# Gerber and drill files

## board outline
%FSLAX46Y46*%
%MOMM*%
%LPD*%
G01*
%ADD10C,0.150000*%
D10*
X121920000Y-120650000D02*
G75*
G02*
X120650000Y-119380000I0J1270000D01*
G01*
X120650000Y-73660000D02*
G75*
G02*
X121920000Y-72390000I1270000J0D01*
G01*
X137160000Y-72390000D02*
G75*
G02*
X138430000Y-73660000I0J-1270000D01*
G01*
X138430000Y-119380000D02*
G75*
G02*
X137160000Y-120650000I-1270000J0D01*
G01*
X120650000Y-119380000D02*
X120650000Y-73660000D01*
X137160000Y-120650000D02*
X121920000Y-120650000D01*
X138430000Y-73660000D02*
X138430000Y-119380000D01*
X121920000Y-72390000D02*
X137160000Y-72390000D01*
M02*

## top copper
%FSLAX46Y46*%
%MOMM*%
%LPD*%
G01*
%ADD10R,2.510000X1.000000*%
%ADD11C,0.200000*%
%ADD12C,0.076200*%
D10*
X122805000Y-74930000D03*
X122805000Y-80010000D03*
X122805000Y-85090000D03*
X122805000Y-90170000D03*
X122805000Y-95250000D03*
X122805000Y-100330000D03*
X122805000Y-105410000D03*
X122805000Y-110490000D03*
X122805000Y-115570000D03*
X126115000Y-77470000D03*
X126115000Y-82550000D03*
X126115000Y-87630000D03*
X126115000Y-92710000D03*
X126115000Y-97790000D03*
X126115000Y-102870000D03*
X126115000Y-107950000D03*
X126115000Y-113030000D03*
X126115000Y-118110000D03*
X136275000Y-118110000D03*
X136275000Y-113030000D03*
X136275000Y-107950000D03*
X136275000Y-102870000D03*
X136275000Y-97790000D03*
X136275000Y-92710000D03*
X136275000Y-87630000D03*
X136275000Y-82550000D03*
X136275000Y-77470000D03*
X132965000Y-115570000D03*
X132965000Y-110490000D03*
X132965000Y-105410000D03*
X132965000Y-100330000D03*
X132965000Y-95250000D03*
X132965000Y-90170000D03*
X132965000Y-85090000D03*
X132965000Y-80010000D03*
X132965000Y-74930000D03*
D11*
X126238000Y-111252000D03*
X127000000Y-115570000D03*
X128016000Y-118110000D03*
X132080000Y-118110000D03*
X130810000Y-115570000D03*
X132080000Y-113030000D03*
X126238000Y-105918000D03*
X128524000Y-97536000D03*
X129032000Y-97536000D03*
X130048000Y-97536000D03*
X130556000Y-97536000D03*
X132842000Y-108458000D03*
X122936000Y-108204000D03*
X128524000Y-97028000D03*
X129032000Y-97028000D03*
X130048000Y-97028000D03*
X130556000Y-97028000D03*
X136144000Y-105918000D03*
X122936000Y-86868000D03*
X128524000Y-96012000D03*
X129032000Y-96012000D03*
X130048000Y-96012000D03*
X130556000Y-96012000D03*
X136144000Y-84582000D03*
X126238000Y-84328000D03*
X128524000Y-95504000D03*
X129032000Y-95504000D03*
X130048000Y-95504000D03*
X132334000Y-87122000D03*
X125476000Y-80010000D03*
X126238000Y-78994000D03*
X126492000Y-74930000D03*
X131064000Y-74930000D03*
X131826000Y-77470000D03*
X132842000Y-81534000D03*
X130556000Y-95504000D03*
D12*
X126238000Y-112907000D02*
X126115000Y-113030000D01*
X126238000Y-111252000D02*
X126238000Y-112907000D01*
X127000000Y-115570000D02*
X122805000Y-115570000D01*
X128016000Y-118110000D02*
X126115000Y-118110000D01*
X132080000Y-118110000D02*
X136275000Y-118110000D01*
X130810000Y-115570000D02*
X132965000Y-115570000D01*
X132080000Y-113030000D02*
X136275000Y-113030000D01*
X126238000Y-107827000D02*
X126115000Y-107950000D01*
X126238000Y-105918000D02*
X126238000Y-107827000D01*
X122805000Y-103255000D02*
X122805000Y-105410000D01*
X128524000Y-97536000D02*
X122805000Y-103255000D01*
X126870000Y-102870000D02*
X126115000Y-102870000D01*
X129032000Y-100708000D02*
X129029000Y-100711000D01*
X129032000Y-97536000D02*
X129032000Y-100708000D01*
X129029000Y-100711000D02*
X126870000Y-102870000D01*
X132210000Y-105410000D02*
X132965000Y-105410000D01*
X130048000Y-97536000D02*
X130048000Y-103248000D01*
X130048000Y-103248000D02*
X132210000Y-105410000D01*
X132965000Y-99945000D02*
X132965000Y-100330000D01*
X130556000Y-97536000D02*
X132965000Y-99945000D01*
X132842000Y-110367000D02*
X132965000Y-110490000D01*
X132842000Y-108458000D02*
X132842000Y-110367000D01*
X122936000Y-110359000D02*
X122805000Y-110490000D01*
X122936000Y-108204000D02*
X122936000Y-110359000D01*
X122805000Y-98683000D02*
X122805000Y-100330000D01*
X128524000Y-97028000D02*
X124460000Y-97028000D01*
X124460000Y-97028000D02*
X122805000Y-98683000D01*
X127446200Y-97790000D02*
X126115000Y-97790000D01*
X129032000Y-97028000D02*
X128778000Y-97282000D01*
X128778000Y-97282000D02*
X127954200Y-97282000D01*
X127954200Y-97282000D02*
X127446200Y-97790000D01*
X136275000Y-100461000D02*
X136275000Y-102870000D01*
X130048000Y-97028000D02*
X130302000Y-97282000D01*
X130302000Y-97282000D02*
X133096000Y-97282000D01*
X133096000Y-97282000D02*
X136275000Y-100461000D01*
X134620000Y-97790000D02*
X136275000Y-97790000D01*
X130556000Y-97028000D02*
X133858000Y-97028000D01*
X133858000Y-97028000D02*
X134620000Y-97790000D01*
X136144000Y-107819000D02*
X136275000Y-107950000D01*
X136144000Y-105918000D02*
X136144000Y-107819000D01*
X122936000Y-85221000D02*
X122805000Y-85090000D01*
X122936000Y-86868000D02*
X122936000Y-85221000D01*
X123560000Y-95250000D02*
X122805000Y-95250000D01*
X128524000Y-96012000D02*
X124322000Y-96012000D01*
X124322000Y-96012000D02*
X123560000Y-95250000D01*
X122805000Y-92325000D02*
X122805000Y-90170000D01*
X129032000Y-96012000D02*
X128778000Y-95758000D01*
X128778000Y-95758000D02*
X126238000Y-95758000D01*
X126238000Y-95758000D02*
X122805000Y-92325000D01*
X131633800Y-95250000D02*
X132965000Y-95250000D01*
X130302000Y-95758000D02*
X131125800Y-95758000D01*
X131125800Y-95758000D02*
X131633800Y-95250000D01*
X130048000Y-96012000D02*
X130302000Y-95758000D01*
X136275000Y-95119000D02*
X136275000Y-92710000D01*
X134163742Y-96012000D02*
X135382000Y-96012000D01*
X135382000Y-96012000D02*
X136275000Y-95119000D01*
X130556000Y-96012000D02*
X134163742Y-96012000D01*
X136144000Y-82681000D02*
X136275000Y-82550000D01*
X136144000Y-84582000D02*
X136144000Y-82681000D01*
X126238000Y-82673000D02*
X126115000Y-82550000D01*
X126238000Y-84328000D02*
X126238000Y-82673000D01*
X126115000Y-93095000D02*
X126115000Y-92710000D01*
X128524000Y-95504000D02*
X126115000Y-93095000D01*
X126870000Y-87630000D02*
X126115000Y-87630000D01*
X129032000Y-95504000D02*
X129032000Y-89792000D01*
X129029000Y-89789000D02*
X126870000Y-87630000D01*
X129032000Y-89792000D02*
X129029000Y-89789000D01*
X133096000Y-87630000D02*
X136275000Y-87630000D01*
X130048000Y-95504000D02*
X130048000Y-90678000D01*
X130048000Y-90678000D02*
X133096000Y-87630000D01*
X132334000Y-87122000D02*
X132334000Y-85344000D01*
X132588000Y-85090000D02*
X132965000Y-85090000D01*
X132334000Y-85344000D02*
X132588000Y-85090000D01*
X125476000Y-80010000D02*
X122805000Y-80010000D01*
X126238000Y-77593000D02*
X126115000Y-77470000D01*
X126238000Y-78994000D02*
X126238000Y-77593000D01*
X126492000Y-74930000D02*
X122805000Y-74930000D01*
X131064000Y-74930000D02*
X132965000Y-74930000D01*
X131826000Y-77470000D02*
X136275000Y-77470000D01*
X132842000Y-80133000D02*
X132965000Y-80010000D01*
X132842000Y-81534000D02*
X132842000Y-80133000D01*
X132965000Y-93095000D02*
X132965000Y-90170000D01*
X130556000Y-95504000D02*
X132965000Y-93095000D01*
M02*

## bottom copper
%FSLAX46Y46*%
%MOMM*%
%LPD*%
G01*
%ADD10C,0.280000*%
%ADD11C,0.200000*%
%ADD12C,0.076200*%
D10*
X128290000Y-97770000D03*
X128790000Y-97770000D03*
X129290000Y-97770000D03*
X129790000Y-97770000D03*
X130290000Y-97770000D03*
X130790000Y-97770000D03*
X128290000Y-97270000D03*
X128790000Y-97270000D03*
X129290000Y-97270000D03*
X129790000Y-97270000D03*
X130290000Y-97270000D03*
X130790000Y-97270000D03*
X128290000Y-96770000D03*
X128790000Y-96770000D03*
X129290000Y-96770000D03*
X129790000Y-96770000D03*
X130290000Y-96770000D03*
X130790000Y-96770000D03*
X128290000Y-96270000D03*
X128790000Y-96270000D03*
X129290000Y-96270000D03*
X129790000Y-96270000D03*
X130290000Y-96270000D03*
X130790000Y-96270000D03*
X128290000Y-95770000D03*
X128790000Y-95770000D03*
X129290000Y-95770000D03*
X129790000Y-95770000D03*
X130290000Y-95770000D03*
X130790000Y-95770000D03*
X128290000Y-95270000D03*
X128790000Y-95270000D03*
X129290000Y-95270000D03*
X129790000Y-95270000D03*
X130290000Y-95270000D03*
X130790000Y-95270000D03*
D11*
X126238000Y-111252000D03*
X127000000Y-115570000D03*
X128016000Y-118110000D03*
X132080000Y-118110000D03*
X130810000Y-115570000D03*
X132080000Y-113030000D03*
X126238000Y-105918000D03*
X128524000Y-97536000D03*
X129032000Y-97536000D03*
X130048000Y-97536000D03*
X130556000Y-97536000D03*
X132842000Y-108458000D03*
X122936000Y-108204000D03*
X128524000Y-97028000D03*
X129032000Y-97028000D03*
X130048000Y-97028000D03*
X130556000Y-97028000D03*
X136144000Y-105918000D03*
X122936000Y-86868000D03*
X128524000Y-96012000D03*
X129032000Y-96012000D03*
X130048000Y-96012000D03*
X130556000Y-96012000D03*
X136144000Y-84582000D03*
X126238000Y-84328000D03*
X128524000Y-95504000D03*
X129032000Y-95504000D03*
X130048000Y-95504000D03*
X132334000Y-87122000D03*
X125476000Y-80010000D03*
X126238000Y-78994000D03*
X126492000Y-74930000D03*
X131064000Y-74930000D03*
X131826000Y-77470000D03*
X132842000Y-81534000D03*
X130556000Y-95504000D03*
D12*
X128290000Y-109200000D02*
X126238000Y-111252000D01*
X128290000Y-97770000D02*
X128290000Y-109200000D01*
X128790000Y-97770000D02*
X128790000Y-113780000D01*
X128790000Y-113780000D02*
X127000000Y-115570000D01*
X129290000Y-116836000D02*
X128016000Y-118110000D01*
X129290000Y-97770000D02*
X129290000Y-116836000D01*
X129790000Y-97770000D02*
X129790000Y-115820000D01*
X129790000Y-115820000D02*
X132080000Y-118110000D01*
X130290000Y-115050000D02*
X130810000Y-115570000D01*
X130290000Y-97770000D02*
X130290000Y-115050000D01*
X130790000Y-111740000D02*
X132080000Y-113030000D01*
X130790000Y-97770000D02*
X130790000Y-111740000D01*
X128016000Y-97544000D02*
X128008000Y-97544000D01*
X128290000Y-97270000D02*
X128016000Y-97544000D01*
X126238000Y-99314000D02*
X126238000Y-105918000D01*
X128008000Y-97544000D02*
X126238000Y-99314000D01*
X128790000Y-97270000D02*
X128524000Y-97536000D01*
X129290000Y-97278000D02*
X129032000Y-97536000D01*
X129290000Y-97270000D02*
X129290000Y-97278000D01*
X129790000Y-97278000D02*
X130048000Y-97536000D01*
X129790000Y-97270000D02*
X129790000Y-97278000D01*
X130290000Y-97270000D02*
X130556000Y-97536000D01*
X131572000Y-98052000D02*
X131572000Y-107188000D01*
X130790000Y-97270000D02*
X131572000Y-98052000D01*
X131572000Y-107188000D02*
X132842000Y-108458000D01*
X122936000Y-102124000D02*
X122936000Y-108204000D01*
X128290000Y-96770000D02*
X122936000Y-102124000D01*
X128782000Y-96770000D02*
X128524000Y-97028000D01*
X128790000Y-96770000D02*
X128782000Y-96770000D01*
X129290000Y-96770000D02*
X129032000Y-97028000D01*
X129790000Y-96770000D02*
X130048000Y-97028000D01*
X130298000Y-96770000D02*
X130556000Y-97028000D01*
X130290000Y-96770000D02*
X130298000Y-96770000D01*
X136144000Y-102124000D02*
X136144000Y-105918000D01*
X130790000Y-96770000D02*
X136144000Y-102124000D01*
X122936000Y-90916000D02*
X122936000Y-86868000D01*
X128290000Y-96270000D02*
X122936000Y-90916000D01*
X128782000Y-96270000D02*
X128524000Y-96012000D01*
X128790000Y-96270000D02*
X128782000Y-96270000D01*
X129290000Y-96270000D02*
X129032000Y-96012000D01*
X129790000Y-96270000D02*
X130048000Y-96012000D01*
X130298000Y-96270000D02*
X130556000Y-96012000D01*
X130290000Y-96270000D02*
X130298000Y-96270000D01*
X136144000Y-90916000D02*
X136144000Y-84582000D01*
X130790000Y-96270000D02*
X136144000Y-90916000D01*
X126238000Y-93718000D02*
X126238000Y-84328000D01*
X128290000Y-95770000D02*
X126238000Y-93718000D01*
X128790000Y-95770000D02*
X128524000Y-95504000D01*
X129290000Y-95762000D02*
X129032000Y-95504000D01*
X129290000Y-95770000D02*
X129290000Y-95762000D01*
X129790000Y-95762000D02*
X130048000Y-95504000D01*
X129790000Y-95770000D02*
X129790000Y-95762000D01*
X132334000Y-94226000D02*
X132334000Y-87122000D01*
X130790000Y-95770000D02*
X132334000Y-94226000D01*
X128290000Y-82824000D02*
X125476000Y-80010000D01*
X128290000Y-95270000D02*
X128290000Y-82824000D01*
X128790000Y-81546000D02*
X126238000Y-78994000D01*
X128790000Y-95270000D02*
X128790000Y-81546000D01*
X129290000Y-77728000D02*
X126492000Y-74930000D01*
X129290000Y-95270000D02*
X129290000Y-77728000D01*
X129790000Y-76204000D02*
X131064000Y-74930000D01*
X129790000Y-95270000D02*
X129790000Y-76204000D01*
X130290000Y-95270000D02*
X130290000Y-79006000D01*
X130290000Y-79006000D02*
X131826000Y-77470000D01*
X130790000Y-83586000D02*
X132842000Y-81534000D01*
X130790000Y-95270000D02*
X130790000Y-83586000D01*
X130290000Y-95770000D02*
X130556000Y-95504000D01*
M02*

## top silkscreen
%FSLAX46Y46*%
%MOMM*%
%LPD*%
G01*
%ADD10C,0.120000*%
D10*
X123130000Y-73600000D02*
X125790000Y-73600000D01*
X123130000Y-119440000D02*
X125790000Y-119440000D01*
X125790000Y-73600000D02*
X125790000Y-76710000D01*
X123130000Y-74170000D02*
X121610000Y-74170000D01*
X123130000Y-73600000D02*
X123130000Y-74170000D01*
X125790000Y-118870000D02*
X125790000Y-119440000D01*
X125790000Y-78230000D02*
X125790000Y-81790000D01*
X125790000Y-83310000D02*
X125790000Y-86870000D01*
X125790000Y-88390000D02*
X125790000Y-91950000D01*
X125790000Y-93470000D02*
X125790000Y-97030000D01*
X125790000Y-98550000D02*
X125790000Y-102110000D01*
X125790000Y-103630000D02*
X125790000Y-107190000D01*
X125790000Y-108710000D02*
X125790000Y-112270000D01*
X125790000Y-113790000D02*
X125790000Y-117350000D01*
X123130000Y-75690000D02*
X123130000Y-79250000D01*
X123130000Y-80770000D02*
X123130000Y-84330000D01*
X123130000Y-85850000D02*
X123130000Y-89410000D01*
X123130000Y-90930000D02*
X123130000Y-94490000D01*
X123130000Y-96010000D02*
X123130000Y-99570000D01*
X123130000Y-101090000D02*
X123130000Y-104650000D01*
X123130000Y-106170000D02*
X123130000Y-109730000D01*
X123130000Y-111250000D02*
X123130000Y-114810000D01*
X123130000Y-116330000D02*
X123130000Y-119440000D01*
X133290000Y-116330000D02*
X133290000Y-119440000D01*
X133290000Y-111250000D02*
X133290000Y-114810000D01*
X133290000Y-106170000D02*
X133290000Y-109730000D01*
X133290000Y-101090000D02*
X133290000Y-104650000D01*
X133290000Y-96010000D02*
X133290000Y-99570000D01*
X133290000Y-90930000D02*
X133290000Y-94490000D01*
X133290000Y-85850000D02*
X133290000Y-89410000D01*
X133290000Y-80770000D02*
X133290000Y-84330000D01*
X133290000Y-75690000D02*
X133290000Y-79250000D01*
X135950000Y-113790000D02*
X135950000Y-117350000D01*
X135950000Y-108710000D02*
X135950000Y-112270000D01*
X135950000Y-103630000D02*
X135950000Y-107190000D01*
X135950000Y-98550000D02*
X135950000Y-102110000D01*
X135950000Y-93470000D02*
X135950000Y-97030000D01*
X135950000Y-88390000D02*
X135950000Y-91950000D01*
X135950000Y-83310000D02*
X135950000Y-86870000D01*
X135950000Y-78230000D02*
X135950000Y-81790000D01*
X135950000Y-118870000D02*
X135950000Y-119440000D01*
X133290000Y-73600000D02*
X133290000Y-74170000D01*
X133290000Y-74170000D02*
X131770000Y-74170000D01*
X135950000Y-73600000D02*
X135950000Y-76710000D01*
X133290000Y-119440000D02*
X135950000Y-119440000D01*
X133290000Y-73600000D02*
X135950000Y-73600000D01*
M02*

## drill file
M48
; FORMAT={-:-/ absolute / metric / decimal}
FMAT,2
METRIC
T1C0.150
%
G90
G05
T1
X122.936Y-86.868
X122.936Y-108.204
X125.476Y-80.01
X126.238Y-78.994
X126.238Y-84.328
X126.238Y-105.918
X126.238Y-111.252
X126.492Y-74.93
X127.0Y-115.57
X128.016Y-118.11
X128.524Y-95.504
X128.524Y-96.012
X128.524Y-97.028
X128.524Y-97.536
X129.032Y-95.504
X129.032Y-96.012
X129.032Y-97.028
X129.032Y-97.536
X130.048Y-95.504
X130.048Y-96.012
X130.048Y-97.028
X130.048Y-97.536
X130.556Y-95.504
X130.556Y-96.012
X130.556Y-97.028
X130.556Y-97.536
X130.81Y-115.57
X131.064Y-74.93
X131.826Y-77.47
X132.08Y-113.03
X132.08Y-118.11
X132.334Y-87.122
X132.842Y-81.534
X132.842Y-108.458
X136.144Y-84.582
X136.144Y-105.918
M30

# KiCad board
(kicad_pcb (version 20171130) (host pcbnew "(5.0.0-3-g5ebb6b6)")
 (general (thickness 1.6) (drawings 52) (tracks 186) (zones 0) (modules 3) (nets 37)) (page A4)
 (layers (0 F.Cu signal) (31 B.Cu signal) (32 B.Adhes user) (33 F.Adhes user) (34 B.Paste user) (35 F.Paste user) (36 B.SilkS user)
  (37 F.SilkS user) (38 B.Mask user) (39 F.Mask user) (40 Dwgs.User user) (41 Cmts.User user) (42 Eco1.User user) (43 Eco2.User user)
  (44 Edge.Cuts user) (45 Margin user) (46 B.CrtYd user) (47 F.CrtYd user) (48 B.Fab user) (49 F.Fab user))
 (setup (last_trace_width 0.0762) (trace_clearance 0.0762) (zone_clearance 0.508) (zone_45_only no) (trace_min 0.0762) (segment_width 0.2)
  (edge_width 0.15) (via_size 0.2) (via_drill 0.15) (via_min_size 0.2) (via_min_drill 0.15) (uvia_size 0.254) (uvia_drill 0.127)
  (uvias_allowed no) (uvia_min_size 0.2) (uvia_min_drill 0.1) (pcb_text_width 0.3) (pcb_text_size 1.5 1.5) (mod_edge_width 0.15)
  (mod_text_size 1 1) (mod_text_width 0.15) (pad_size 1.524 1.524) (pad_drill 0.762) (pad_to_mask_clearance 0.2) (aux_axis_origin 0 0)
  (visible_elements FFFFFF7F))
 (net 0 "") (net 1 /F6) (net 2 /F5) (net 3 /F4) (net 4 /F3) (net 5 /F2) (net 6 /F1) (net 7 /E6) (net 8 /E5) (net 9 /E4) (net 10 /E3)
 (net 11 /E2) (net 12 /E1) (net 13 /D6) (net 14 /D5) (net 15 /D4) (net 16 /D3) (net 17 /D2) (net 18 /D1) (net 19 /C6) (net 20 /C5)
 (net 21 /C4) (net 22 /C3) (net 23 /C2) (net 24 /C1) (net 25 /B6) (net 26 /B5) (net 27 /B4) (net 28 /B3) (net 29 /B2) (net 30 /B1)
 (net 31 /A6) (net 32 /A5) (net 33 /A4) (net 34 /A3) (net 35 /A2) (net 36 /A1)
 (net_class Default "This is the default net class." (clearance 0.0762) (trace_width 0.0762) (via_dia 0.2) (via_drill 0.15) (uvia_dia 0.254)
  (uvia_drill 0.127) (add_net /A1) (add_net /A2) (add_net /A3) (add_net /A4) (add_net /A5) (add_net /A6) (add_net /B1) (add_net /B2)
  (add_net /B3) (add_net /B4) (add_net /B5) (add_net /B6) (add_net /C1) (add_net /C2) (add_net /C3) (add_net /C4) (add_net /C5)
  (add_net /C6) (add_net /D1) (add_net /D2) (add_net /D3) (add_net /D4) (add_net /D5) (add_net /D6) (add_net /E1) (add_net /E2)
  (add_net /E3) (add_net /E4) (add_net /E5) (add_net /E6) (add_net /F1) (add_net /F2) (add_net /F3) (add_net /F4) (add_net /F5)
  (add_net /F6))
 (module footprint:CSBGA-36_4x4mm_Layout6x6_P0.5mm (layer B.Cu) (at 129.54 96.52 180)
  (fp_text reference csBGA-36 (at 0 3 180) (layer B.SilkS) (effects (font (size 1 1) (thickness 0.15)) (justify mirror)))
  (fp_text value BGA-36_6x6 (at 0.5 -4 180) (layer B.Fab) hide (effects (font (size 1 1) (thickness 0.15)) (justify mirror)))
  (pad F6 smd circle (at 1.25 -1.25 180) (size 0.28 0.28) (layers B.Cu B.Paste B.Mask) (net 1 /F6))
  (pad F5 smd circle (at 0.75 -1.25 180) (size 0.28 0.28) (layers B.Cu B.Paste B.Mask) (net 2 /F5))
  (pad F4 smd circle (at 0.25 -1.25 180) (size 0.28 0.28) (layers B.Cu B.Paste B.Mask) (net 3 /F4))
  (pad F3 smd circle (at -0.25 -1.25 180) (size 0.28 0.28) (layers B.Cu B.Paste B.Mask) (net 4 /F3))
  (pad F2 smd circle (at -0.75 -1.25 180) (size 0.28 0.28) (layers B.Cu B.Paste B.Mask) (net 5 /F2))
  (pad F1 smd circle (at -1.25 -1.25 180) (size 0.28 0.28) (layers B.Cu B.Paste B.Mask) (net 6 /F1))
  (pad E6 smd circle (at 1.25 -0.75 180) (size 0.28 0.28) (layers B.Cu B.Paste B.Mask) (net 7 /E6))
  (pad E5 smd circle (at 0.75 -0.75 180) (size 0.28 0.28) (layers B.Cu B.Paste B.Mask) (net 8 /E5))
  (pad E4 smd circle (at 0.25 -0.75 180) (size 0.28 0.28) (layers B.Cu B.Paste B.Mask) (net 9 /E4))
  (pad E3 smd circle (at -0.25 -0.75 180) (size 0.28 0.28) (layers B.Cu B.Paste B.Mask) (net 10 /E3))
  (pad E2 smd circle (at -0.75 -0.75 180) (size 0.28 0.28) (layers B.Cu B.Paste B.Mask) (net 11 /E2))
  (pad E1 smd circle (at -1.25 -0.75 180) (size 0.28 0.28) (layers B.Cu B.Paste B.Mask) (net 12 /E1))
  (pad D6 smd circle (at 1.25 -0.25 180) (size 0.28 0.28) (layers B.Cu B.Paste B.Mask) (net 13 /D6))
  (pad D5 smd circle (at 0.75 -0.25 180) (size 0.28 0.28) (layers B.Cu B.Paste B.Mask) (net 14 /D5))
  (pad D4 smd circle (at 0.25 -0.25 180) (size 0.28 0.28) (layers B.Cu B.Paste B.Mask) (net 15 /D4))
  (pad D3 smd circle (at -0.25 -0.25 180) (size 0.28 0.28) (layers B.Cu B.Paste B.Mask) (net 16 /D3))
  (pad D2 smd circle (at -0.75 -0.25 180) (size 0.28 0.28) (layers B.Cu B.Paste B.Mask) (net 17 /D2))
  (pad D1 smd circle (at -1.25 -0.25 180) (size 0.28 0.28) (layers B.Cu B.Paste B.Mask) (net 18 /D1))
  (pad C6 smd circle (at 1.25 0.25 180) (size 0.28 0.28) (layers B.Cu B.Paste B.Mask) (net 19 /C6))
  (pad C5 smd circle (at 0.75 0.25 180) (size 0.28 0.28) (layers B.Cu B.Paste B.Mask) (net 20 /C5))
  (pad C4 smd circle (at 0.25 0.25 180) (size 0.28 0.28) (layers B.Cu B.Paste B.Mask) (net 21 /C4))
  (pad C3 smd circle (at -0.25 0.25 180) (size 0.28 0.28) (layers B.Cu B.Paste B.Mask) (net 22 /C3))
  (pad C2 smd circle (at -0.75 0.25 180) (size 0.28 0.28) (layers B.Cu B.Paste B.Mask) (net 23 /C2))
  (pad C1 smd circle (at -1.25 0.25 180) (size 0.28 0.28) (layers B.Cu B.Paste B.Mask) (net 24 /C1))
  (pad B6 smd circle (at 1.25 0.75 180) (size 0.28 0.28) (layers B.Cu B.Paste B.Mask) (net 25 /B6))
  (pad B5 smd circle (at 0.75 0.75 180) (size 0.28 0.28) (layers B.Cu B.Paste B.Mask) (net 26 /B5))
  (pad B4 smd circle (at 0.25 0.75 180) (size 0.28 0.28) (layers B.Cu B.Paste B.Mask) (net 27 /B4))
  (pad B3 smd circle (at -0.25 0.75 180) (size 0.28 0.28) (layers B.Cu B.Paste B.Mask) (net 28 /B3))
  (pad B2 smd circle (at -0.75 0.75 180) (size 0.28 0.28) (layers B.Cu B.Paste B.Mask) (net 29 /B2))
  (pad B1 smd circle (at -1.25 0.75 180) (size 0.28 0.28) (layers B.Cu B.Paste B.Mask) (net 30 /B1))
  (pad A6 smd circle (at 1.25 1.25 180) (size 0.28 0.28) (layers B.Cu B.Paste B.Mask) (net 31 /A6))
  (pad A5 smd circle (at 0.75 1.25 180) (size 0.28 0.28) (layers B.Cu B.Paste B.Mask) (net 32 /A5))
  (pad A4 smd circle (at 0.25 1.25 180) (size 0.28 0.28) (layers B.Cu B.Paste B.Mask) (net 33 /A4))
  (pad A3 smd circle (at -0.25 1.25 180) (size 0.28 0.28) (layers B.Cu B.Paste B.Mask) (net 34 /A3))
  (pad A2 smd circle (at -0.75 1.25 180) (size 0.28 0.28) (layers B.Cu B.Paste B.Mask) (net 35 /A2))
  (pad A1 smd circle (at -1.25 1.25 180) (size 0.28 0.28) (layers B.Cu B.Paste B.Mask) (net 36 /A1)))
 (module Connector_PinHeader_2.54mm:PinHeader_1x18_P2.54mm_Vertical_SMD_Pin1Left (layer F.Cu) (at 124.46 96.52)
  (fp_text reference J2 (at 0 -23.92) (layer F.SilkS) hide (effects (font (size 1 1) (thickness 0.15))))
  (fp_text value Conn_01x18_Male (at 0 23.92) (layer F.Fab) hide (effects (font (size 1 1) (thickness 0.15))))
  (fp_line (start -1.33 -22.92) (end 1.33 -22.92) (layer F.SilkS) (width 0.12))
  (fp_line (start -1.33 22.92) (end 1.33 22.92) (layer F.SilkS) (width 0.12))
  (fp_line (start 1.33 -22.92) (end 1.33 -19.81) (layer F.SilkS) (width 0.12))
  (fp_line (start -1.33 -22.35) (end -2.85 -22.35) (layer F.SilkS) (width 0.12))
  (fp_line (start -1.33 -22.92) (end -1.33 -22.35) (layer F.SilkS) (width 0.12))
  (fp_line (start 1.33 22.35) (end 1.33 22.92) (layer F.SilkS) (width 0.12))
  (fp_line (start 1.33 -18.29) (end 1.33 -14.73) (layer F.SilkS) (width 0.12))
  (fp_line (start 1.33 -13.21) (end 1.33 -9.65) (layer F.SilkS) (width 0.12))
  (fp_line (start 1.33 -8.13) (end 1.33 -4.57) (layer F.SilkS) (width 0.12))
  (fp_line (start 1.33 -3.05) (end 1.33 0.51) (layer F.SilkS) (width 0.12))
  (fp_line (start 1.33 2.03) (end 1.33 5.59) (layer F.SilkS) (width 0.12))
  (fp_line (start 1.33 7.11) (end 1.33 10.67) (layer F.SilkS) (width 0.12))
  (fp_line (start 1.33 12.19) (end 1.33 15.75) (layer F.SilkS) (width 0.12))
  (fp_line (start 1.33 17.27) (end 1.33 20.83) (layer F.SilkS) (width 0.12))
  (fp_line (start -1.33 -20.83) (end -1.33 -17.27) (layer F.SilkS) (width 0.12))
  (fp_line (start -1.33 -15.75) (end -1.33 -12.19) (layer F.SilkS) (width 0.12))
  (fp_line (start -1.33 -10.67) (end -1.33 -7.11) (layer F.SilkS) (width 0.12))
  (fp_line (start -1.33 -5.59) (end -1.33 -2.03) (layer F.SilkS) (width 0.12))
  (fp_line (start -1.33 -0.51) (end -1.33 3.05) (layer F.SilkS) (width 0.12))
  (fp_line (start -1.33 4.57) (end -1.33 8.13) (layer F.SilkS) (width 0.12))
  (fp_line (start -1.33 9.65) (end -1.33 13.21) (layer F.SilkS) (width 0.12))
  (fp_line (start -1.33 14.73) (end -1.33 18.29) (layer F.SilkS) (width 0.12))
  (fp_line (start -1.33 19.81) (end -1.33 22.92) (layer F.SilkS) (width 0.12))
  (pad 1 smd rect (at -1.655 -21.59) (size 2.51 1) (layers F.Cu F.Paste F.Mask) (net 33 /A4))
  (pad 3 smd rect (at -1.655 -16.51) (size 2.51 1) (layers F.Cu F.Paste F.Mask) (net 31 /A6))
  (pad 5 smd rect (at -1.655 -11.43) (size 2.51 1) (layers F.Cu F.Paste F.Mask) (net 19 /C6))
  (pad 7 smd rect (at -1.655 -6.35) (size 2.51 1) (layers F.Cu F.Paste F.Mask) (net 21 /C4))
  (pad 9 smd rect (at -1.655 -1.27) (size 2.51 1) (layers F.Cu F.Paste F.Mask) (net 20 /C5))
  (pad 11 smd rect (at -1.655 3.81) (size 2.51 1) (layers F.Cu F.Paste F.Mask) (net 14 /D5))
  (pad 13 smd rect (at -1.655 8.89) (size 2.51 1) (layers F.Cu F.Paste F.Mask) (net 8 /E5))
  (pad 15 smd rect (at -1.655 13.97) (size 2.51 1) (layers F.Cu F.Paste F.Mask) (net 13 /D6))
  (pad 17 smd rect (at -1.655 19.05) (size 2.51 1) (layers F.Cu F.Paste F.Mask) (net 2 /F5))
  (pad 2 smd rect (at 1.655 -19.05) (size 2.51 1) (layers F.Cu F.Paste F.Mask) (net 32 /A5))
  (pad 4 smd rect (at 1.655 -13.97) (size 2.51 1) (layers F.Cu F.Paste F.Mask) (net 25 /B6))
  (pad 6 smd rect (at 1.655 -8.89) (size 2.51 1) (layers F.Cu F.Paste F.Mask) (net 27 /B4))
  (pad 8 smd rect (at 1.655 -3.81) (size 2.51 1) (layers F.Cu F.Paste F.Mask) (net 26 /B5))
  (pad 10 smd rect (at 1.655 1.27) (size 2.51 1) (layers F.Cu F.Paste F.Mask) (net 15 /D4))
  (pad 12 smd rect (at 1.655 6.35) (size 2.51 1) (layers F.Cu F.Paste F.Mask) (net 9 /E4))
  (pad 14 smd rect (at 1.655 11.43) (size 2.51 1) (layers F.Cu F.Paste F.Mask) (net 7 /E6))
  (pad 16 smd rect (at 1.655 16.51) (size 2.51 1) (layers F.Cu F.Paste F.Mask) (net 1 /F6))
  (pad 18 smd rect (at 1.655 21.59) (size 2.51 1) (layers F.Cu F.Paste F.Mask) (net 3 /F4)))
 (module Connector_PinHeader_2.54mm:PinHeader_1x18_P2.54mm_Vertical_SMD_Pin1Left (layer F.Cu) (at 134.62 96.52)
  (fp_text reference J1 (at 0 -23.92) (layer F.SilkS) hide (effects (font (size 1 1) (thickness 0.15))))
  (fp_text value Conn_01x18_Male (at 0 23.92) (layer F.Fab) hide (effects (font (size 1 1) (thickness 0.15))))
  (fp_line (start -1.33 19.81) (end -1.33 22.92) (layer F.SilkS) (width 0.12))
  (fp_line (start -1.33 14.73) (end -1.33 18.29) (layer F.SilkS) (width 0.12))
  (fp_line (start -1.33 9.65) (end -1.33 13.21) (layer F.SilkS) (width 0.12))
  (fp_line (start -1.33 4.57) (end -1.33 8.13) (layer F.SilkS) (width 0.12))
  (fp_line (start -1.33 -0.51) (end -1.33 3.05) (layer F.SilkS) (width 0.12))
  (fp_line (start -1.33 -5.59) (end -1.33 -2.03) (layer F.SilkS) (width 0.12))
  (fp_line (start -1.33 -10.67) (end -1.33 -7.11) (layer F.SilkS) (width 0.12))
  (fp_line (start -1.33 -15.75) (end -1.33 -12.19) (layer F.SilkS) (width 0.12))
  (fp_line (start -1.33 -20.83) (end -1.33 -17.27) (layer F.SilkS) (width 0.12))
  (fp_line (start 1.33 17.27) (end 1.33 20.83) (layer F.SilkS) (width 0.12))
  (fp_line (start 1.33 12.19) (end 1.33 15.75) (layer F.SilkS) (width 0.12))
  (fp_line (start 1.33 7.11) (end 1.33 10.67) (layer F.SilkS) (width 0.12))
  (fp_line (start 1.33 2.03) (end 1.33 5.59) (layer F.SilkS) (width 0.12))
  (fp_line (start 1.33 -3.05) (end 1.33 0.51) (layer F.SilkS) (width 0.12))
  (fp_line (start 1.33 -8.13) (end 1.33 -4.57) (layer F.SilkS) (width 0.12))
  (fp_line (start 1.33 -13.21) (end 1.33 -9.65) (layer F.SilkS) (width 0.12))
  (fp_line (start 1.33 -18.29) (end 1.33 -14.73) (layer F.SilkS) (width 0.12))
  (fp_line (start 1.33 22.35) (end 1.33 22.92) (layer F.SilkS) (width 0.12))
  (fp_line (start -1.33 -22.92) (end -1.33 -22.35) (layer F.SilkS) (width 0.12))
  (fp_line (start -1.33 -22.35) (end -2.85 -22.35) (layer F.SilkS) (width 0.12))
  (fp_line (start 1.33 -22.92) (end 1.33 -19.81) (layer F.SilkS) (width 0.12))
  (fp_line (start -1.33 22.92) (end 1.33 22.92) (layer F.SilkS) (width 0.12))
  (fp_line (start -1.33 -22.92) (end 1.33 -22.92) (layer F.SilkS) (width 0.12))
  (pad 18 smd rect (at 1.655 21.59) (size 2.51 1) (layers F.Cu F.Paste F.Mask) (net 4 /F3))
  (pad 16 smd rect (at 1.655 16.51) (size 2.51 1) (layers F.Cu F.Paste F.Mask) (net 6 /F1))
  (pad 14 smd rect (at 1.655 11.43) (size 2.51 1) (layers F.Cu F.Paste F.Mask) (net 18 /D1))
  (pad 12 smd rect (at 1.655 6.35) (size 2.51 1) (layers F.Cu F.Paste F.Mask) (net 16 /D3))
  (pad 10 smd rect (at 1.655 1.27) (size 2.51 1) (layers F.Cu F.Paste F.Mask) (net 17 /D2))
  (pad 8 smd rect (at 1.655 -3.81) (size 2.51 1) (layers F.Cu F.Paste F.Mask) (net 23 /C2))
  (pad 6 smd rect (at 1.655 -8.89) (size 2.51 1) (layers F.Cu F.Paste F.Mask) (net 28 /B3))
  (pad 4 smd rect (at 1.655 -13.97) (size 2.51 1) (layers F.Cu F.Paste F.Mask) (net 24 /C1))
  (pad 2 smd rect (at 1.655 -19.05) (size 2.51 1) (layers F.Cu F.Paste F.Mask) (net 35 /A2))
  (pad 17 smd rect (at -1.655 19.05) (size 2.51 1) (layers F.Cu F.Paste F.Mask) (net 5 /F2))
  (pad 15 smd rect (at -1.655 13.97) (size 2.51 1) (layers F.Cu F.Paste F.Mask) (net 12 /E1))
  (pad 13 smd rect (at -1.655 8.89) (size 2.51 1) (layers F.Cu F.Paste F.Mask) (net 10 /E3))
  (pad 11 smd rect (at -1.655 3.81) (size 2.51 1) (layers F.Cu F.Paste F.Mask) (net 11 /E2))
  (pad 9 smd rect (at -1.655 -1.27) (size 2.51 1) (layers F.Cu F.Paste F.Mask) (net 22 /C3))
  (pad 7 smd rect (at -1.655 -6.35) (size 2.51 1) (layers F.Cu F.Paste F.Mask) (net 29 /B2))
  (pad 5 smd rect (at -1.655 -11.43) (size 2.51 1) (layers F.Cu F.Paste F.Mask) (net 30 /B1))
  (pad 3 smd rect (at -1.655 -16.51) (size 2.51 1) (layers F.Cu F.Paste F.Mask) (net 36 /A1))
  (pad 1 smd rect (at -1.655 -21.59) (size 2.51 1) (layers F.Cu F.Paste F.Mask) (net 34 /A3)))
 (gr_arc (start 121.92 119.38) (end 120.65 119.38) (angle -90) (layer Edge.Cuts) (width 0.15))
 (gr_arc (start 121.92 73.66) (end 121.92 72.39) (angle -90) (layer Edge.Cuts) (width 0.15))
 (gr_arc (start 137.16 73.66) (end 138.43 73.66) (angle -90) (layer Edge.Cuts) (width 0.15))
 (gr_arc (start 137.16 119.38) (end 137.16 120.65) (angle -90) (layer Edge.Cuts) (width 0.15))
 (gr_line (start 120.65 119.38) (end 120.65 73.66) (layer Edge.Cuts) (width 0.15))
 (gr_line (start 137.16 120.65) (end 121.92 120.65) (layer Edge.Cuts) (width 0.15))
 (gr_line (start 138.43 73.66) (end 138.43 119.38) (layer Edge.Cuts) (width 0.15))
 (gr_line (start 121.92 72.39) (end 137.16 72.39) (layer Edge.Cuts) (width 0.15))
 (via (at 126.238 111.252) (size 0.2) (drill 0.15) (layers F.Cu B.Cu) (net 1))
 (segment (start 128.29 109.2) (end 126.238 111.252) (width 0.0762) (layer B.Cu) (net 1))
 (segment (start 128.29 97.77) (end 128.29 109.2) (width 0.0762) (layer B.Cu) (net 1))
 (segment (start 126.238 112.907) (end 126.115 113.03) (width 0.0762) (layer F.Cu) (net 1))
 (segment (start 126.238 111.252) (end 126.238 112.907) (width 0.0762) (layer F.Cu) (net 1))
 (segment (start 128.79 97.77) (end 128.79 113.78) (width 0.0762) (layer B.Cu) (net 2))
 (via (at 127 115.57) (size 0.2) (drill 0.15) (layers F.Cu B.Cu) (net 2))
 (segment (start 128.79 113.78) (end 127 115.57) (width 0.0762) (layer B.Cu) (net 2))
 (segment (start 127 115.57) (end 122.805 115.57) (width 0.0762) (layer F.Cu) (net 2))
 (segment (start 129.29 116.836) (end 128.016 118.11) (width 0.0762) (layer B.Cu) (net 3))
 (via (at 128.016 118.11) (size 0.2) (drill 0.15) (layers F.Cu B.Cu) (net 3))
 (segment (start 129.29 97.77) (end 129.29 116.836) (width 0.0762) (layer B.Cu) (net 3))
 (segment (start 128.016 118.11) (end 126.115 118.11) (width 0.0762) (layer F.Cu) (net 3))
 (segment (start 129.79 97.77) (end 129.79 115.82) (width 0.0762) (layer B.Cu) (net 4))
 (via (at 132.08 118.11) (size 0.2) (drill 0.15) (layers F.Cu B.Cu) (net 4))
 (segment (start 129.79 115.82) (end 132.08 118.11) (width 0.0762) (layer B.Cu) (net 4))
 (segment (start 132.08 118.11) (end 136.275 118.11) (width 0.0762) (layer F.Cu) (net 4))
 (via (at 130.81 115.57) (size 0.2) (drill 0.15) (layers F.Cu B.Cu) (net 5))
 (segment (start 130.29 115.05) (end 130.81 115.57) (width 0.0762) (layer B.Cu) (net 5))
 (segment (start 130.29 97.77) (end 130.29 115.05) (width 0.0762) (layer B.Cu) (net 5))
 (segment (start 130.81 115.57) (end 132.965 115.57) (width 0.0762) (layer F.Cu) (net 5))
 (segment (start 130.79 111.74) (end 132.08 113.03) (width 0.0762) (layer B.Cu) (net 6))
 (via (at 132.08 113.03) (size 0.2) (drill 0.15) (layers F.Cu B.Cu) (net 6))
 (segment (start 130.79 97.77) (end 130.79 111.74) (width 0.0762) (layer B.Cu) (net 6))
 (segment (start 132.08 113.03) (end 136.275 113.03) (width 0.0762) (layer F.Cu) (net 6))
 (segment (start 128.016 97.544) (end 128.008 97.544) (width 0.0762) (layer B.Cu) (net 7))
 (segment (start 128.29 97.27) (end 128.016 97.544) (width 0.0762) (layer B.Cu) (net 7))
 (via (at 126.238 105.918) (size 0.2) (drill 0.15) (layers F.Cu B.Cu) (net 7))
 (segment (start 126.238 99.314) (end 126.238 105.918) (width 0.0762) (layer B.Cu) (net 7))
 (segment (start 128.008 97.544) (end 126.238 99.314) (width 0.0762) (layer B.Cu) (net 7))
 (segment (start 126.238 107.827) (end 126.115 107.95) (width 0.0762) (layer F.Cu) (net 7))
 (segment (start 126.238 105.918) (end 126.238 107.827) (width 0.0762) (layer F.Cu) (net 7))
 (via (at 128.524 97.536) (size 0.2) (drill 0.15) (layers F.Cu B.Cu) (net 8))
 (segment (start 128.79 97.27) (end 128.524 97.536) (width 0.0762) (layer B.Cu) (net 8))
 (segment (start 122.805 103.255) (end 122.805 105.41) (width 0.0762) (layer F.Cu) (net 8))
 (segment (start 128.524 97.536) (end 122.805 103.255) (width 0.0762) (layer F.Cu) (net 8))
 (segment (start 126.87 102.87) (end 126.115 102.87) (width 0.0762) (layer F.Cu) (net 9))
 (via (at 129.032 97.536) (size 0.2) (drill 0.15) (layers F.Cu B.Cu) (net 9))
 (segment (start 129.29 97.278) (end 129.032 97.536) (width 0.0762) (layer B.Cu) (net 9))
 (segment (start 129.29 97.27) (end 129.29 97.278) (width 0.0762) (layer B.Cu) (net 9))
 (segment (start 129.032 100.708) (end 129.029 100.711) (width 0.0762) (layer F.Cu) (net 9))
 (segment (start 129.032 97.536) (end 129.032 100.708) (width 0.0762) (layer F.Cu) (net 9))
 (segment (start 129.029 100.711) (end 126.87 102.87) (width 0.0762) (layer F.Cu) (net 9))
 (segment (start 132.21 105.41) (end 132.965 105.41) (width 0.0762) (layer F.Cu) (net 10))
 (via (at 130.048 97.536) (size 0.2) (drill 0.15) (layers F.Cu B.Cu) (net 10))
 (segment (start 129.79 97.278) (end 130.048 97.536) (width 0.0762) (layer B.Cu) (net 10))
 (segment (start 129.79 97.27) (end 129.79 97.278) (width 0.0762) (layer B.Cu) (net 10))
 (segment (start 130.048 97.536) (end 130.048 103.248) (width 0.0762) (layer F.Cu) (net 10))
 (segment (start 130.048 103.248) (end 132.21 105.41) (width 0.0762) (layer F.Cu) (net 10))
 (via (at 130.556 97.536) (size 0.2) (drill 0.15) (layers F.Cu B.Cu) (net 11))
 (segment (start 130.29 97.27) (end 130.556 97.536) (width 0.0762) (layer B.Cu) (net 11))
 (segment (start 132.965 99.945) (end 132.965 100.33) (width 0.0762) (layer F.Cu) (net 11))
 (segment (start 130.556 97.536) (end 132.965 99.945) (width 0.0762) (layer F.Cu) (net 11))
 (segment (start 131.572 98.052) (end 131.572 107.188) (width 0.0762) (layer B.Cu) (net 12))
 (segment (start 130.79 97.27) (end 131.572 98.052) (width 0.0762) (layer B.Cu) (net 12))
 (via (at 132.842 108.458) (size 0.2) (drill 0.15) (layers F.Cu B.Cu) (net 12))
 (segment (start 131.572 107.188) (end 132.842 108.458) (width 0.0762) (layer B.Cu) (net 12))
 (segment (start 132.842 110.367) (end 132.965 110.49) (width 0.0762) (layer F.Cu) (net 12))
 (segment (start 132.842 108.458) (end 132.842 110.367) (width 0.0762) (layer F.Cu) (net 12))
 (via (at 122.936 108.204) (size 0.2) (drill 0.15) (layers F.Cu B.Cu) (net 13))
 (segment (start 122.936 102.124) (end 122.936 108.204) (width 0.0762) (layer B.Cu) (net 13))
 (segment (start 128.29 96.77) (end 122.936 102.124) (width 0.0762) (layer B.Cu) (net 13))
 (segment (start 122.936 110.359) (end 122.805 110.49) (width 0.0762) (layer F.Cu) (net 13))
 (segment (start 122.936 108.204) (end 122.936 110.359) (width 0.0762) (layer F.Cu) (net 13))
 (segment (start 122.805 98.683) (end 122.805 100.33) (width 0.0762) (layer F.Cu) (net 14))
 (segment (start 128.782 96.77) (end 128.524 97.028) (width 0.0762) (layer B.Cu) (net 14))
 (via (at 128.524 97.028) (size 0.2) (drill 0.15) (layers F.Cu B.Cu) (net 14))
 (segment (start 128.79 96.77) (end 128.782 96.77) (width 0.0762) (layer B.Cu) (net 14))
 (segment (start 128.524 97.028) (end 124.46 97.028) (width 0.0762) (layer F.Cu) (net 14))
 (segment (start 124.46 97.028) (end 122.805 98.683) (width 0.0762) (layer F.Cu) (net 14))
 (via (at 129.032 97.028) (size 0.2) (drill 0.15) (layers F.Cu B.Cu) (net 15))
 (segment (start 129.29 96.77) (end 129.032 97.028) (width 0.0762) (layer B.Cu) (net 15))
 (segment (start 127.4462 97.79) (end 126.115 97.79) (width 0.0762) (layer F.Cu) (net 15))
 (segment (start 129.032 97.028) (end 128.778 97.282) (width 0.0762) (layer F.Cu) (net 15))
 (segment (start 128.778 97.282) (end 127.9542 97.282) (width 0.0762) (layer F.Cu) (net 15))
 (segment (start 127.9542 97.282) (end 127.4462 97.79) (width 0.0762) (layer F.Cu) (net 15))
 (via (at 130.048 97.028) (size 0.2) (drill 0.15) (layers F.Cu B.Cu) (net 16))
 (segment (start 129.79 96.77) (end 130.048 97.028) (width 0.0762) (layer B.Cu) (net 16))
 (segment (start 136.275 100.461) (end 136.275 102.87) (width 0.0762) (layer F.Cu) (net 16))
 (segment (start 130.048 97.028) (end 130.302 97.282) (width 0.0762) (layer F.Cu) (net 16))
 (segment (start 130.302 97.282) (end 133.096 97.282) (width 0.0762) (layer F.Cu) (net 16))
 (segment (start 133.096 97.282) (end 136.275 100.461) (width 0.0762) (layer F.Cu) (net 16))
 (segment (start 134.62 97.79) (end 136.275 97.79) (width 0.0762) (layer F.Cu) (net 17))
 (via (at 130.556 97.028) (size 0.2) (drill 0.15) (layers F.Cu B.Cu) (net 17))
 (segment (start 130.298 96.77) (end 130.556 97.028) (width 0.0762) (layer B.Cu) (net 17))
 (segment (start 130.29 96.77) (end 130.298 96.77) (width 0.0762) (layer B.Cu) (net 17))
 (segment (start 130.556 97.028) (end 133.858 97.028) (width 0.0762) (layer F.Cu) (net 17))
 (segment (start 133.858 97.028) (end 134.62 97.79) (width 0.0762) (layer F.Cu) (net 17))
 (via (at 136.144 105.918) (size 0.2) (drill 0.15) (layers F.Cu B.Cu) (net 18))
 (segment (start 136.144 102.124) (end 136.144 105.918) (width 0.0762) (layer B.Cu) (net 18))
 (segment (start 130.79 96.77) (end 136.144 102.124) (width 0.0762) (layer B.Cu) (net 18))
 (segment (start 136.144 107.819) (end 136.275 107.95) (width 0.0762) (layer F.Cu) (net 18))
 (segment (start 136.144 105.918) (end 136.144 107.819) (width 0.0762) (layer F.Cu) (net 18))
 (via (at 122.936 86.868) (size 0.2) (drill 0.15) (layers F.Cu B.Cu) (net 19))
 (segment (start 122.936 90.916) (end 122.936 86.868) (width 0.0762) (layer B.Cu) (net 19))
 (segment (start 128.29 96.27) (end 122.936 90.916) (width 0.0762) (layer B.Cu) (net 19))
 (segment (start 122.936 85.221) (end 122.805 85.09) (width 0.0762) (layer F.Cu) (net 19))
 (segment (start 122.936 86.868) (end 122.936 85.221) (width 0.0762) (layer F.Cu) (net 19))
 (segment (start 123.56 95.25) (end 122.805 95.25) (width 0.0762) (layer F.Cu) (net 20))
 (via (at 128.524 96.012) (size 0.2) (drill 0.15) (layers F.Cu B.Cu) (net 20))
 (segment (start 128.782 96.27) (end 128.524 96.012) (width 0.0762) (layer B.Cu) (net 20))
 (segment (start 128.79 96.27) (end 128.782 96.27) (width 0.0762) (layer B.Cu) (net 20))
 (segment (start 128.524 96.012) (end 124.322 96.012) (width 0.0762) (layer F.Cu) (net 20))
 (segment (start 124.322 96.012) (end 123.56 95.25) (width 0.0762) (layer F.Cu) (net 20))
 (segment (start 122.805 92.325) (end 122.805 90.17) (width 0.0762) (layer F.Cu) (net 21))
 (via (at 129.032 96.012) (size 0.2) (drill 0.15) (layers F.Cu B.Cu) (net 21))
 (segment (start 129.29 96.27) (end 129.032 96.012) (width 0.0762) (layer B.Cu) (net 21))
 (segment (start 129.032 96.012) (end 128.778 95.758) (width 0.0762) (layer F.Cu) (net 21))
 (segment (start 128.778 95.758) (end 126.238 95.758) (width 0.0762) (layer F.Cu) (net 21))
 (segment (start 126.238 95.758) (end 122.805 92.325) (width 0.0762) (layer F.Cu) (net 21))
 (segment (start 131.6338 95.25) (end 132.965 95.25) (width 0.0762) (layer F.Cu) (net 22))
 (via (at 130.048 96.012) (size 0.2) (drill 0.15) (layers F.Cu B.Cu) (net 22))
 (segment (start 129.79 96.27) (end 130.048 96.012) (width 0.0762) (layer B.Cu) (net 22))
 (segment (start 130.302 95.758) (end 131.1258 95.758) (width 0.0762) (layer F.Cu) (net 22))
 (segment (start 131.1258 95.758) (end 131.6338 95.25) (width 0.0762) (layer F.Cu) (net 22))
 (segment (start 130.048 96.012) (end 130.302 95.758) (width 0.0762) (layer F.Cu) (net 22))
 (segment (start 136.275 95.119) (end 136.275 92.71) (width 0.0762) (layer F.Cu) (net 23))
 (via (at 130.556 96.012) (size 0.2) (drill 0.15) (layers F.Cu B.Cu) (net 23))
 (segment (start 130.298 96.27) (end 130.556 96.012) (width 0.0762) (layer B.Cu) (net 23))
 (segment (start 130.29 96.27) (end 130.298 96.27) (width 0.0762) (layer B.Cu) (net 23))
 (segment (start 134.163742 96.012) (end 135.382 96.012) (width 0.0762) (layer F.Cu) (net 23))
 (segment (start 135.382 96.012) (end 136.275 95.119) (width 0.0762) (layer F.Cu) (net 23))
 (segment (start 130.556 96.012) (end 134.163742 96.012) (width 0.0762) (layer F.Cu) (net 23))
 (via (at 136.144 84.582) (size 0.2) (drill 0.15) (layers F.Cu B.Cu) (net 24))
 (segment (start 136.144 90.916) (end 136.144 84.582) (width 0.0762) (layer B.Cu) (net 24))
 (segment (start 130.79 96.27) (end 136.144 90.916) (width 0.0762) (layer B.Cu) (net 24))
 (segment (start 136.144 82.681) (end 136.275 82.55) (width 0.0762) (layer F.Cu) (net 24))
 (segment (start 136.144 84.582) (end 136.144 82.681) (width 0.0762) (layer F.Cu) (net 24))
 (via (at 126.238 84.328) (size 0.2) (drill 0.15) (layers F.Cu B.Cu) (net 25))
 (segment (start 126.238 93.718) (end 126.238 84.328) (width 0.0762) (layer B.Cu) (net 25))
 (segment (start 128.29 95.77) (end 126.238 93.718) (width 0.0762) (layer B.Cu) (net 25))
 (segment (start 126.238 82.673) (end 126.115 82.55) (width 0.0762) (layer F.Cu) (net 25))
 (segment (start 126.238 84.328) (end 126.238 82.673) (width 0.0762) (layer F.Cu) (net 25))
 (via (at 128.524 95.504) (size 0.2) (drill 0.15) (layers F.Cu B.Cu) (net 26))
 (segment (start 128.79 95.77) (end 128.524 95.504) (width 0.0762) (layer B.Cu) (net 26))
 (segment (start 126.115 93.095) (end 126.115 92.71) (width 0.0762) (layer F.Cu) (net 26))
 (segment (start 128.524 95.504) (end 126.115 93.095) (width 0.0762) (layer F.Cu) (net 26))
 (segment (start 126.87 87.63) (end 126.115 87.63) (width 0.0762) (layer F.Cu) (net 27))
 (via (at 129.032 95.504) (size 0.2) (drill 0.15) (layers F.Cu B.Cu) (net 27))
 (segment (start 129.29 95.762) (end 129.032 95.504) (width 0.0762) (layer B.Cu) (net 27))
 (segment (start 129.29 95.77) (end 129.29 95.762) (width 0.0762) (layer B.Cu) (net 27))
 (segment (start 129.032 95.504) (end 129.032 89.792) (width 0.0762) (layer F.Cu) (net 27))
 (segment (start 129.029 89.789) (end 126.87 87.63) (width 0.0762) (layer F.Cu) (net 27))
 (segment (start 129.032 89.792) (end 129.029 89.789) (width 0.0762) (layer F.Cu) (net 27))
 (segment (start 133.096 87.63) (end 136.275 87.63) (width 0.0762) (layer F.Cu) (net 28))
 (via (at 130.048 95.504) (size 0.2) (drill 0.15) (layers F.Cu B.Cu) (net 28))
 (segment (start 129.79 95.762) (end 130.048 95.504) (width 0.0762) (layer B.Cu) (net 28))
 (segment (start 129.79 95.77) (end 129.79 95.762) (width 0.0762) (layer B.Cu) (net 28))
 (segment (start 130.048 95.504) (end 130.048 90.678) (width 0.0762) (layer F.Cu) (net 28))
 (segment (start 130.048 90.678) (end 133.096 87.63) (width 0.0762) (layer F.Cu) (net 28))
 (via (at 132.334 87.122) (size 0.2) (drill 0.15) (layers F.Cu B.Cu) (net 30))
 (segment (start 132.334 94.226) (end 132.334 87.122) (width 0.0762) (layer B.Cu) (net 30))
 (segment (start 130.79 95.77) (end 132.334 94.226) (width 0.0762) (layer B.Cu) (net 30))
 (segment (start 132.334 87.122) (end 132.334 85.344) (width 0.0762) (layer F.Cu) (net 30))
 (segment (start 132.588 85.09) (end 132.965 85.09) (width 0.0762) (layer F.Cu) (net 30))
 (segment (start 132.334 85.344) (end 132.588 85.09) (width 0.0762) (layer F.Cu) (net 30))
 (via (at 125.476 80.01) (size 0.2) (drill 0.15) (layers F.Cu B.Cu) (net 31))
 (segment (start 128.29 82.824) (end 125.476 80.01) (width 0.0762) (layer B.Cu) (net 31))
 (segment (start 128.29 95.27) (end 128.29 82.824) (width 0.0762) (layer B.Cu) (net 31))
 (segment (start 125.476 80.01) (end 122.805 80.01) (width 0.0762) (layer F.Cu) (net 31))
 (segment (start 128.79 81.546) (end 126.238 78.994) (width 0.0762) (layer B.Cu) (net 32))
 (via (at 126.238 78.994) (size 0.2) (drill 0.15) (layers F.Cu B.Cu) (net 32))
 (segment (start 128.79 95.27) (end 128.79 81.546) (width 0.0762) (layer B.Cu) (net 32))
 (segment (start 126.238 77.593) (end 126.115 77.47) (width 0.0762) (layer F.Cu) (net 32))
 (segment (start 126.238 78.994) (end 126.238 77.593) (width 0.0762) (layer F.Cu) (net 32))
 (via (at 126.492 74.93) (size 0.2) (drill 0.15) (layers F.Cu B.Cu) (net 33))
 (segment (start 129.29 77.728) (end 126.492 74.93) (width 0.0762) (layer B.Cu) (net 33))
 (segment (start 129.29 95.27) (end 129.29 77.728) (width 0.0762) (layer B.Cu) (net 33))
 (segment (start 126.492 74.93) (end 122.805 74.93) (width 0.0762) (layer F.Cu) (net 33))
 (via (at 131.064 74.93) (size 0.2) (drill 0.15) (layers F.Cu B.Cu) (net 34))
 (segment (start 129.79 76.204) (end 131.064 74.93) (width 0.0762) (layer B.Cu) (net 34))
 (segment (start 129.79 95.27) (end 129.79 76.204) (width 0.0762) (layer B.Cu) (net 34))
 (segment (start 131.064 74.93) (end 132.965 74.93) (width 0.0762) (layer F.Cu) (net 34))
 (segment (start 130.29 95.27) (end 130.29 79.006) (width 0.0762) (layer B.Cu) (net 35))
 (via (at 131.826 77.47) (size 0.2) (drill 0.15) (layers F.Cu B.Cu) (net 35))
 (segment (start 130.29 79.006) (end 131.826 77.47) (width 0.0762) (layer B.Cu) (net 35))
 (segment (start 131.826 77.47) (end 136.275 77.47) (width 0.0762) (layer F.Cu) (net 35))
 (via (at 132.842 81.534) (size 0.2) (drill 0.15) (layers F.Cu B.Cu) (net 36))
 (segment (start 130.79 83.586) (end 132.842 81.534) (width 0.0762) (layer B.Cu) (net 36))
 (segment (start 130.79 95.27) (end 130.79 83.586) (width 0.0762) (layer B.Cu) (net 36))
 (segment (start 132.842 80.133) (end 132.965 80.01) (width 0.0762) (layer F.Cu) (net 36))
 (segment (start 132.842 81.534) (end 132.842 80.133) (width 0.0762) (layer F.Cu) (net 36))
 (segment (start 132.965 93.095) (end 132.965 90.17) (width 0.0762) (layer F.Cu) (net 29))
 (via (at 130.556 95.504) (size 0.2) (drill 0.15) (layers F.Cu B.Cu) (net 29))
 (segment (start 130.29 95.77) (end 130.556 95.504) (width 0.0762) (layer B.Cu) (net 29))
 (segment (start 130.556 95.504) (end 132.965 93.095) (width 0.0762) (layer F.Cu) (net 29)))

